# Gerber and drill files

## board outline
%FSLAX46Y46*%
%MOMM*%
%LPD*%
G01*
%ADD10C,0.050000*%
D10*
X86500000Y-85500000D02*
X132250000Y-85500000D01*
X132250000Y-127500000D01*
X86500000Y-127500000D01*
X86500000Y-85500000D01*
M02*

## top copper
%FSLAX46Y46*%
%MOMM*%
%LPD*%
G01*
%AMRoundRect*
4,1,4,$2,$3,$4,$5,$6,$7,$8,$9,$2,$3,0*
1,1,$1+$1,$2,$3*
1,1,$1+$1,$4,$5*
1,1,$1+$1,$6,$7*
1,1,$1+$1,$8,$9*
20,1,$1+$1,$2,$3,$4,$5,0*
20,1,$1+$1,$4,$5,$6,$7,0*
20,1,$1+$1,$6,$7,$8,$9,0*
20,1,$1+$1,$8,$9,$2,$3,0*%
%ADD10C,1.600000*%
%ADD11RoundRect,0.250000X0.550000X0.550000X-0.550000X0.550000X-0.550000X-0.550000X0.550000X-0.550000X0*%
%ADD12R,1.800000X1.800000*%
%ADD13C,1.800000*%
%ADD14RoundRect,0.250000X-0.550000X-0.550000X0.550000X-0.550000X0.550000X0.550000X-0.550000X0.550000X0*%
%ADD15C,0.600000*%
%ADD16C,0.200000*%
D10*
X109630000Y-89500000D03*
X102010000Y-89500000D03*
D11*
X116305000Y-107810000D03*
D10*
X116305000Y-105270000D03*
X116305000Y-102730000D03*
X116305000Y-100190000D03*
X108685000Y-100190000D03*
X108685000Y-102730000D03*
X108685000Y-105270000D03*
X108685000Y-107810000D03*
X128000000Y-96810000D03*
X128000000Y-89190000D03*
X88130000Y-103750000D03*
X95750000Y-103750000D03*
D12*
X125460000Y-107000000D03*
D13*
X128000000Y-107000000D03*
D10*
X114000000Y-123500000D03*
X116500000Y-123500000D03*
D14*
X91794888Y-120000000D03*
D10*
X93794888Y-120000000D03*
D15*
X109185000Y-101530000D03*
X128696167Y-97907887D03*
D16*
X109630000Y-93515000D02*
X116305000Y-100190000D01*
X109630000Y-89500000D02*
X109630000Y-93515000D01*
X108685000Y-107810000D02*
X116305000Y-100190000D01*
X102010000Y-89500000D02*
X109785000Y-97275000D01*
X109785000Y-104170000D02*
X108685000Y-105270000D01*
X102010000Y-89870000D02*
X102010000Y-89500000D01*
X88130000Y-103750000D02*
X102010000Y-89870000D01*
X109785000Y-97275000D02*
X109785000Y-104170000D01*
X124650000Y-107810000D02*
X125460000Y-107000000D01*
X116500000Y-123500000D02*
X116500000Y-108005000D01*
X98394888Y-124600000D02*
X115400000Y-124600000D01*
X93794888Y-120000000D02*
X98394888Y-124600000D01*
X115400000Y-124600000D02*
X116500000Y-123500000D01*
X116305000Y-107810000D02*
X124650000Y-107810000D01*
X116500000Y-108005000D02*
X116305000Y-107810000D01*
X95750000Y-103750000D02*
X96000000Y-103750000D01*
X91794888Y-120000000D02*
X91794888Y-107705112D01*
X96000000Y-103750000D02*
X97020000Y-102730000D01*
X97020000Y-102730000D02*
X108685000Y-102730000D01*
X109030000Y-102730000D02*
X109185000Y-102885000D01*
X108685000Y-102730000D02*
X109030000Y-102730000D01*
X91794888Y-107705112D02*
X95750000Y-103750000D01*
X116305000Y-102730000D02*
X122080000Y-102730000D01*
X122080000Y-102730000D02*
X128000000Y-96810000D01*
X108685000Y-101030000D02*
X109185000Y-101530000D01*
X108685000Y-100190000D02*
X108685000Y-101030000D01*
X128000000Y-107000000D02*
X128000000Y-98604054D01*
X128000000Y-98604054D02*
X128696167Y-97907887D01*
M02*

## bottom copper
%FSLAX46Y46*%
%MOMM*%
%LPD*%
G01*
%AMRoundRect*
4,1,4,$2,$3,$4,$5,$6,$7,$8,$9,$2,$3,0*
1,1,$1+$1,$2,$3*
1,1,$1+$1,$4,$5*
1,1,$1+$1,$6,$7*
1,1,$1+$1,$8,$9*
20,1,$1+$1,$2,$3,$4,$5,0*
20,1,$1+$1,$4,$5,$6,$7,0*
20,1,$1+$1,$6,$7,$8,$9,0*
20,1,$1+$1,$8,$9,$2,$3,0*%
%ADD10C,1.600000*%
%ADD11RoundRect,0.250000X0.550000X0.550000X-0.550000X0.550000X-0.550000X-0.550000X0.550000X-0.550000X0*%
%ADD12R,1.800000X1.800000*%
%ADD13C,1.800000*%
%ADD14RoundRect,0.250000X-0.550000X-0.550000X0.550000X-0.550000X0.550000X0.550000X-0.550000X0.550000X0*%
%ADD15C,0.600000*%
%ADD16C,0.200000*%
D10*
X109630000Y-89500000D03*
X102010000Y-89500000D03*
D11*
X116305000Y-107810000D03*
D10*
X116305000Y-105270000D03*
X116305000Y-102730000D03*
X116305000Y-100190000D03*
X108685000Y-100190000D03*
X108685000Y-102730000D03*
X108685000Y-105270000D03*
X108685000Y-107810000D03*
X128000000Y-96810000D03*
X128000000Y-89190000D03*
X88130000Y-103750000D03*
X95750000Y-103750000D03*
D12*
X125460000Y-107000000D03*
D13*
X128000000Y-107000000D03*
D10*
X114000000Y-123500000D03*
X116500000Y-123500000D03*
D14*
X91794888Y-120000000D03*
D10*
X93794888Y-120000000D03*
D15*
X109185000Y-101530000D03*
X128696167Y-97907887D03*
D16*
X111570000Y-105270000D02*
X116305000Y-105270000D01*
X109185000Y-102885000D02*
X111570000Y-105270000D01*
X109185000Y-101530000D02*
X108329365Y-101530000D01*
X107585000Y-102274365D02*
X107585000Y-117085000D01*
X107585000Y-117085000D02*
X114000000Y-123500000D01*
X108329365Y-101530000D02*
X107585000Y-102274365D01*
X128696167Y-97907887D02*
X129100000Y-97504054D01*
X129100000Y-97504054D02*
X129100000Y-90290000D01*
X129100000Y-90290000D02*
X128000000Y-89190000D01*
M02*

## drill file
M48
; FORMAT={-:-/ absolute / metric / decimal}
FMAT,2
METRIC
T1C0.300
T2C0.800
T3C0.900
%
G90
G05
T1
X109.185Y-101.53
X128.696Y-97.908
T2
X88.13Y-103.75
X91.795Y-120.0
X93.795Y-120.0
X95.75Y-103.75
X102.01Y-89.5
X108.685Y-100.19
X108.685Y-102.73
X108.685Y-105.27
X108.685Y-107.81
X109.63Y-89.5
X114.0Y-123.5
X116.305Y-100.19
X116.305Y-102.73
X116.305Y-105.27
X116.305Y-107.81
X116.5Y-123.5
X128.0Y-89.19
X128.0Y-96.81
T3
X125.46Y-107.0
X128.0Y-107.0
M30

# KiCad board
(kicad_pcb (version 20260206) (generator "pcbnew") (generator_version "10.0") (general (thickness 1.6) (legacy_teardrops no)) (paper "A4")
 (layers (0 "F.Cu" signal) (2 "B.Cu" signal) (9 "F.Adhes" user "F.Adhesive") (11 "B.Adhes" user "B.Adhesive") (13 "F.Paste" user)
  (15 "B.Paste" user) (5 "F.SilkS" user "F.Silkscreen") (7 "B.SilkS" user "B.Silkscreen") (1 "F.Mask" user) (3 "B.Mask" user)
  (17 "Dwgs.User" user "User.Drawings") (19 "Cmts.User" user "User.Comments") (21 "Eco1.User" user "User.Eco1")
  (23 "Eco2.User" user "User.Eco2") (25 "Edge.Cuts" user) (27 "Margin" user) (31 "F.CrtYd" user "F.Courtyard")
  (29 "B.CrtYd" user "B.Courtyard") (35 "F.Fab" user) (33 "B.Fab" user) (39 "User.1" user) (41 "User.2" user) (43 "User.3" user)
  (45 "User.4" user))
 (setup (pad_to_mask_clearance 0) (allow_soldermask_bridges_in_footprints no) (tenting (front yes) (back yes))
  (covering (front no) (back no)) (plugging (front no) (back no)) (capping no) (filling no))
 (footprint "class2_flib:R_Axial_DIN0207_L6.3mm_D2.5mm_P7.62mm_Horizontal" (layer "F.Cu") (at 109.63 89.5 180)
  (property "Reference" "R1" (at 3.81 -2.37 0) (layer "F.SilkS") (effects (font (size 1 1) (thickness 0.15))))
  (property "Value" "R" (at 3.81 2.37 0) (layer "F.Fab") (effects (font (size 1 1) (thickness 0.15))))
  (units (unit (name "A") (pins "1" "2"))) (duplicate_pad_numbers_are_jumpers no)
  (pad "1" thru_hole circle (at 0 0 180) (size 1.6 1.6) (drill 0.8) (layers "*.Cu" "*.Mask") (remove_unused_layers no) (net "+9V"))
  (pad "2" thru_hole circle (at 7.62 0 180) (size 1.6 1.6) (drill 0.8) (layers "*.Cu" "*.Mask") (remove_unused_layers no)
   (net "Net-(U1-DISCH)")))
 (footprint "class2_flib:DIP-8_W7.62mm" (layer "F.Cu") (at 116.305 107.81 180)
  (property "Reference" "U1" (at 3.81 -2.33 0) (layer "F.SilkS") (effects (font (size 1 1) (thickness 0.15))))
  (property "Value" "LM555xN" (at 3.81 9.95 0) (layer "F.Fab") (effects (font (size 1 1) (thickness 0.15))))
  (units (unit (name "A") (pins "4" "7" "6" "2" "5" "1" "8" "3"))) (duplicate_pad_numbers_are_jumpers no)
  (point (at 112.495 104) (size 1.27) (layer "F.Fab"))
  (pad "1" thru_hole roundrect (at 0 0 180) (size 1.6 1.6) (drill 0.8) (layers "*.Cu" "*.Mask") (remove_unused_layers no)
   (roundrect_rratio 0.15625) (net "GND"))
  (pad "2" thru_hole circle (at 0 2.54 180) (size 1.6 1.6) (drill 0.8) (layers "*.Cu" "*.Mask") (remove_unused_layers no)
   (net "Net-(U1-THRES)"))
  (pad "3" thru_hole circle (at 0 5.08 180) (size 1.6 1.6) (drill 0.8) (layers "*.Cu" "*.Mask") (remove_unused_layers no)
   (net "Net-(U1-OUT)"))
  (pad "4" thru_hole circle (at 0 7.62 180) (size 1.6 1.6) (drill 0.8) (layers "*.Cu" "*.Mask") (remove_unused_layers no) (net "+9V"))
  (pad "5" thru_hole circle (at 7.62 7.62 180) (size 1.6 1.6) (drill 0.8) (layers "*.Cu" "*.Mask") (remove_unused_layers no)
   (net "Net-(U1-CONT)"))
  (pad "6" thru_hole circle (at 7.62 5.08 180) (size 1.6 1.6) (drill 0.8) (layers "*.Cu" "*.Mask") (remove_unused_layers no)
   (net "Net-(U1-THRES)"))
  (pad "7" thru_hole circle (at 7.62 2.54 180) (size 1.6 1.6) (drill 0.8) (layers "*.Cu" "*.Mask") (remove_unused_layers no)
   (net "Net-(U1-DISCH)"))
  (pad "8" thru_hole circle (at 7.62 0 180) (size 1.6 1.6) (drill 0.8) (layers "*.Cu" "*.Mask") (remove_unused_layers no) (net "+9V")))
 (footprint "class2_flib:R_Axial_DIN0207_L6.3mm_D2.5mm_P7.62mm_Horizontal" (layer "F.Cu") (at 128 96.81 90)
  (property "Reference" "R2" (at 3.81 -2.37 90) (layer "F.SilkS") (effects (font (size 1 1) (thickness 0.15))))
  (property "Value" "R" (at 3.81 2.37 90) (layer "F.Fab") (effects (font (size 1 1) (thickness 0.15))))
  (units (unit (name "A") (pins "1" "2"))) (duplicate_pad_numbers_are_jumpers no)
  (pad "1" thru_hole circle (at 0 0 90) (size 1.6 1.6) (drill 0.8) (layers "*.Cu" "*.Mask") (remove_unused_layers no) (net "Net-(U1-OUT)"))
  (pad "2" thru_hole circle (at 7.62 0 90) (size 1.6 1.6) (drill 0.8) (layers "*.Cu" "*.Mask") (remove_unused_layers no) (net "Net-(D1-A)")))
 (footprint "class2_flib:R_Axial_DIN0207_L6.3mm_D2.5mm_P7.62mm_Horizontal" (layer "F.Cu") (at 88.13 103.75)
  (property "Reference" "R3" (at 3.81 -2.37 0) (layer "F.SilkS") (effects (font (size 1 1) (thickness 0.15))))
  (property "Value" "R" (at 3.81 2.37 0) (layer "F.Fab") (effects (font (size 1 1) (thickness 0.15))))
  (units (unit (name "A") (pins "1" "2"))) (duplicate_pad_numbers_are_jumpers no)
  (pad "1" thru_hole circle (at 0 0) (size 1.6 1.6) (drill 0.8) (layers "*.Cu" "*.Mask") (remove_unused_layers no) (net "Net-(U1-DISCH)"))
  (pad "2" thru_hole circle (at 7.62 0) (size 1.6 1.6) (drill 0.8) (layers "*.Cu" "*.Mask") (remove_unused_layers no) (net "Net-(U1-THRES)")))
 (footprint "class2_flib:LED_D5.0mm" (layer "F.Cu") (at 125.46 107)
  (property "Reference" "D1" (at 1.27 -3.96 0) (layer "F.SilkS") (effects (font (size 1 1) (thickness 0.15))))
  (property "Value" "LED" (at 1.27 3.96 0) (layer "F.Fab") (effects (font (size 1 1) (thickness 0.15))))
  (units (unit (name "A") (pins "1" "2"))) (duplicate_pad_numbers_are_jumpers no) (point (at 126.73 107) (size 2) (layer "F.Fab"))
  (pad "1" thru_hole rect (at 0 0) (size 1.8 1.8) (drill 0.9) (layers "*.Cu" "*.Mask") (remove_unused_layers no) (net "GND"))
  (pad "2" thru_hole circle (at 2.54 0) (size 1.8 1.8) (drill 0.9) (layers "*.Cu" "*.Mask") (remove_unused_layers no) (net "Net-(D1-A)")))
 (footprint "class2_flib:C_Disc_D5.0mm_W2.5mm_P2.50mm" (layer "F.Cu") (at 114 123.5)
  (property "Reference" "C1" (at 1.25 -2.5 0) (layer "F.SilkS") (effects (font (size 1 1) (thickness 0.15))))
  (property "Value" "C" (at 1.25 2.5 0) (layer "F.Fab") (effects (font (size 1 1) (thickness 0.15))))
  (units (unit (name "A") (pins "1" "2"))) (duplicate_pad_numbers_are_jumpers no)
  (pad "1" thru_hole circle (at 0 0) (size 1.6 1.6) (drill 0.8) (layers "*.Cu" "*.Mask") (remove_unused_layers no) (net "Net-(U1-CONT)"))
  (pad "2" thru_hole circle (at 2.5 0) (size 1.6 1.6) (drill 0.8) (layers "*.Cu" "*.Mask") (remove_unused_layers no) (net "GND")))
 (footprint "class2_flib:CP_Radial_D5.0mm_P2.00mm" (layer "F.Cu") (at 91.794888 120)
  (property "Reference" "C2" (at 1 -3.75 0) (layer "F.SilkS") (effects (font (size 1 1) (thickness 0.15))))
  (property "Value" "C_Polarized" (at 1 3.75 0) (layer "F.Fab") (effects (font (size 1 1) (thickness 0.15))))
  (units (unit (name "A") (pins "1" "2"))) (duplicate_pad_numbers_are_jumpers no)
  (pad "1" thru_hole roundrect (at 0 0) (size 1.6 1.6) (drill 0.8) (layers "*.Cu" "*.Mask") (remove_unused_layers no)
   (roundrect_rratio 0.15625) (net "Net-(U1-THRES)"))
  (pad "2" thru_hole circle (at 2 0) (size 1.6 1.6) (drill 0.8) (layers "*.Cu" "*.Mask") (remove_unused_layers no) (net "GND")))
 (gr_rect (start 86.5 85.5) (end 132.25 127.5) (stroke (width 0.05) (type default)) (fill no) (layer "Edge.Cuts"))
 (segment (start 109.63 93.515) (end 116.305 100.19) (width 0.2) (layer "F.Cu") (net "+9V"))
 (segment (start 109.63 89.5) (end 109.63 93.515) (width 0.2) (layer "F.Cu") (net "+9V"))
 (segment (start 108.685 107.81) (end 116.305 100.19) (width 0.2) (layer "F.Cu") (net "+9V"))
 (segment (start 102.01 89.5) (end 109.785 97.275) (width 0.2) (layer "F.Cu") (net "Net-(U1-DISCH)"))
 (segment (start 109.785 104.17) (end 108.685 105.27) (width 0.2) (layer "F.Cu") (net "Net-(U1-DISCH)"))
 (segment (start 102.01 89.87) (end 102.01 89.5) (width 0.2) (layer "F.Cu") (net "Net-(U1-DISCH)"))
 (segment (start 88.13 103.75) (end 102.01 89.87) (width 0.2) (layer "F.Cu") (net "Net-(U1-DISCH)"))
 (segment (start 109.785 97.275) (end 109.785 104.17) (width 0.2) (layer "F.Cu") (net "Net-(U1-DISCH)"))
 (segment (start 124.65 107.81) (end 125.46 107) (width 0.2) (layer "F.Cu") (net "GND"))
 (segment (start 116.5 123.5) (end 116.5 108.005) (width 0.2) (layer "F.Cu") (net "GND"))
 (segment (start 98.394888 124.6) (end 115.4 124.6) (width 0.2) (layer "F.Cu") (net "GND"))
 (segment (start 93.794888 120) (end 98.394888 124.6) (width 0.2) (layer "F.Cu") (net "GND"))
 (segment (start 115.4 124.6) (end 116.5 123.5) (width 0.2) (layer "F.Cu") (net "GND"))
 (segment (start 116.305 107.81) (end 124.65 107.81) (width 0.2) (layer "F.Cu") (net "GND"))
 (segment (start 116.5 108.005) (end 116.305 107.81) (width 0.2) (layer "F.Cu") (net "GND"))
 (segment (start 95.75 103.75) (end 96 103.75) (width 0.2) (layer "F.Cu") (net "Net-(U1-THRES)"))
 (segment (start 91.794888 120) (end 91.794888 107.705112) (width 0.2) (layer "F.Cu") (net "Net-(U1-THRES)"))
 (segment (start 96 103.75) (end 97.02 102.73) (width 0.2) (layer "F.Cu") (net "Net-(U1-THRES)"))
 (segment (start 97.02 102.73) (end 108.685 102.73) (width 0.2) (layer "F.Cu") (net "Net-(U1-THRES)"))
 (segment (start 109.03 102.73) (end 109.185 102.885) (width 0.2) (layer "F.Cu") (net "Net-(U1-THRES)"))
 (segment (start 108.685 102.73) (end 109.03 102.73) (width 0.2) (layer "F.Cu") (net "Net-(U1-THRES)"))
 (segment (start 91.794888 107.705112) (end 95.75 103.75) (width 0.2) (layer "F.Cu") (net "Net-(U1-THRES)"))
 (segment (start 111.57 105.27) (end 116.305 105.27) (width 0.2) (layer "B.Cu") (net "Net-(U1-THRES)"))
 (segment (start 109.185 102.885) (end 111.57 105.27) (width 0.2) (layer "B.Cu") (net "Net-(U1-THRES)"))
 (segment (start 116.305 102.73) (end 122.08 102.73) (width 0.2) (layer "F.Cu") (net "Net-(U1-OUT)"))
 (segment (start 122.08 102.73) (end 128 96.81) (width 0.2) (layer "F.Cu") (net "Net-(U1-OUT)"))
 (segment (start 108.685 101.03) (end 109.185 101.53) (width 0.2) (layer "F.Cu") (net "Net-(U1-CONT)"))
 (segment (start 108.685 100.19) (end 108.685 101.03) (width 0.2) (layer "F.Cu") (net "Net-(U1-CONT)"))
 (via (at 109.185 101.53) (size 0.6) (drill 0.3) (layers "F.Cu" "B.Cu") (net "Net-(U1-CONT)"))
 (segment (start 109.185 101.53) (end 108.329365 101.53) (width 0.2) (layer "B.Cu") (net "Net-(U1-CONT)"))
 (segment (start 107.585 102.274365) (end 107.585 117.085) (width 0.2) (layer "B.Cu") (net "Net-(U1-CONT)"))
 (segment (start 107.585 117.085) (end 114 123.5) (width 0.2) (layer "B.Cu") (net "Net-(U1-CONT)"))
 (segment (start 108.329365 101.53) (end 107.585 102.274365) (width 0.2) (layer "B.Cu") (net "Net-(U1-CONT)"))
 (segment (start 128 107) (end 128 98.604054) (width 0.2) (layer "F.Cu") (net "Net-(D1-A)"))
 (segment (start 128 98.604054) (end 128.696167 97.907887) (width 0.2) (layer "F.Cu") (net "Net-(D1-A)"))
 (via (at 128.696167 97.907887) (size 0.6) (drill 0.3) (layers "F.Cu" "B.Cu") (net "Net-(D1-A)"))
 (segment (start 128.696167 97.907887) (end 129.1 97.504054) (width 0.2) (layer "B.Cu") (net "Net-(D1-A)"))
 (segment (start 129.1 97.504054) (end 129.1 90.29) (width 0.2) (layer "B.Cu") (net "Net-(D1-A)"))
 (segment (start 129.1 90.29) (end 128 89.19) (width 0.2) (layer "B.Cu") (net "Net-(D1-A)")))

